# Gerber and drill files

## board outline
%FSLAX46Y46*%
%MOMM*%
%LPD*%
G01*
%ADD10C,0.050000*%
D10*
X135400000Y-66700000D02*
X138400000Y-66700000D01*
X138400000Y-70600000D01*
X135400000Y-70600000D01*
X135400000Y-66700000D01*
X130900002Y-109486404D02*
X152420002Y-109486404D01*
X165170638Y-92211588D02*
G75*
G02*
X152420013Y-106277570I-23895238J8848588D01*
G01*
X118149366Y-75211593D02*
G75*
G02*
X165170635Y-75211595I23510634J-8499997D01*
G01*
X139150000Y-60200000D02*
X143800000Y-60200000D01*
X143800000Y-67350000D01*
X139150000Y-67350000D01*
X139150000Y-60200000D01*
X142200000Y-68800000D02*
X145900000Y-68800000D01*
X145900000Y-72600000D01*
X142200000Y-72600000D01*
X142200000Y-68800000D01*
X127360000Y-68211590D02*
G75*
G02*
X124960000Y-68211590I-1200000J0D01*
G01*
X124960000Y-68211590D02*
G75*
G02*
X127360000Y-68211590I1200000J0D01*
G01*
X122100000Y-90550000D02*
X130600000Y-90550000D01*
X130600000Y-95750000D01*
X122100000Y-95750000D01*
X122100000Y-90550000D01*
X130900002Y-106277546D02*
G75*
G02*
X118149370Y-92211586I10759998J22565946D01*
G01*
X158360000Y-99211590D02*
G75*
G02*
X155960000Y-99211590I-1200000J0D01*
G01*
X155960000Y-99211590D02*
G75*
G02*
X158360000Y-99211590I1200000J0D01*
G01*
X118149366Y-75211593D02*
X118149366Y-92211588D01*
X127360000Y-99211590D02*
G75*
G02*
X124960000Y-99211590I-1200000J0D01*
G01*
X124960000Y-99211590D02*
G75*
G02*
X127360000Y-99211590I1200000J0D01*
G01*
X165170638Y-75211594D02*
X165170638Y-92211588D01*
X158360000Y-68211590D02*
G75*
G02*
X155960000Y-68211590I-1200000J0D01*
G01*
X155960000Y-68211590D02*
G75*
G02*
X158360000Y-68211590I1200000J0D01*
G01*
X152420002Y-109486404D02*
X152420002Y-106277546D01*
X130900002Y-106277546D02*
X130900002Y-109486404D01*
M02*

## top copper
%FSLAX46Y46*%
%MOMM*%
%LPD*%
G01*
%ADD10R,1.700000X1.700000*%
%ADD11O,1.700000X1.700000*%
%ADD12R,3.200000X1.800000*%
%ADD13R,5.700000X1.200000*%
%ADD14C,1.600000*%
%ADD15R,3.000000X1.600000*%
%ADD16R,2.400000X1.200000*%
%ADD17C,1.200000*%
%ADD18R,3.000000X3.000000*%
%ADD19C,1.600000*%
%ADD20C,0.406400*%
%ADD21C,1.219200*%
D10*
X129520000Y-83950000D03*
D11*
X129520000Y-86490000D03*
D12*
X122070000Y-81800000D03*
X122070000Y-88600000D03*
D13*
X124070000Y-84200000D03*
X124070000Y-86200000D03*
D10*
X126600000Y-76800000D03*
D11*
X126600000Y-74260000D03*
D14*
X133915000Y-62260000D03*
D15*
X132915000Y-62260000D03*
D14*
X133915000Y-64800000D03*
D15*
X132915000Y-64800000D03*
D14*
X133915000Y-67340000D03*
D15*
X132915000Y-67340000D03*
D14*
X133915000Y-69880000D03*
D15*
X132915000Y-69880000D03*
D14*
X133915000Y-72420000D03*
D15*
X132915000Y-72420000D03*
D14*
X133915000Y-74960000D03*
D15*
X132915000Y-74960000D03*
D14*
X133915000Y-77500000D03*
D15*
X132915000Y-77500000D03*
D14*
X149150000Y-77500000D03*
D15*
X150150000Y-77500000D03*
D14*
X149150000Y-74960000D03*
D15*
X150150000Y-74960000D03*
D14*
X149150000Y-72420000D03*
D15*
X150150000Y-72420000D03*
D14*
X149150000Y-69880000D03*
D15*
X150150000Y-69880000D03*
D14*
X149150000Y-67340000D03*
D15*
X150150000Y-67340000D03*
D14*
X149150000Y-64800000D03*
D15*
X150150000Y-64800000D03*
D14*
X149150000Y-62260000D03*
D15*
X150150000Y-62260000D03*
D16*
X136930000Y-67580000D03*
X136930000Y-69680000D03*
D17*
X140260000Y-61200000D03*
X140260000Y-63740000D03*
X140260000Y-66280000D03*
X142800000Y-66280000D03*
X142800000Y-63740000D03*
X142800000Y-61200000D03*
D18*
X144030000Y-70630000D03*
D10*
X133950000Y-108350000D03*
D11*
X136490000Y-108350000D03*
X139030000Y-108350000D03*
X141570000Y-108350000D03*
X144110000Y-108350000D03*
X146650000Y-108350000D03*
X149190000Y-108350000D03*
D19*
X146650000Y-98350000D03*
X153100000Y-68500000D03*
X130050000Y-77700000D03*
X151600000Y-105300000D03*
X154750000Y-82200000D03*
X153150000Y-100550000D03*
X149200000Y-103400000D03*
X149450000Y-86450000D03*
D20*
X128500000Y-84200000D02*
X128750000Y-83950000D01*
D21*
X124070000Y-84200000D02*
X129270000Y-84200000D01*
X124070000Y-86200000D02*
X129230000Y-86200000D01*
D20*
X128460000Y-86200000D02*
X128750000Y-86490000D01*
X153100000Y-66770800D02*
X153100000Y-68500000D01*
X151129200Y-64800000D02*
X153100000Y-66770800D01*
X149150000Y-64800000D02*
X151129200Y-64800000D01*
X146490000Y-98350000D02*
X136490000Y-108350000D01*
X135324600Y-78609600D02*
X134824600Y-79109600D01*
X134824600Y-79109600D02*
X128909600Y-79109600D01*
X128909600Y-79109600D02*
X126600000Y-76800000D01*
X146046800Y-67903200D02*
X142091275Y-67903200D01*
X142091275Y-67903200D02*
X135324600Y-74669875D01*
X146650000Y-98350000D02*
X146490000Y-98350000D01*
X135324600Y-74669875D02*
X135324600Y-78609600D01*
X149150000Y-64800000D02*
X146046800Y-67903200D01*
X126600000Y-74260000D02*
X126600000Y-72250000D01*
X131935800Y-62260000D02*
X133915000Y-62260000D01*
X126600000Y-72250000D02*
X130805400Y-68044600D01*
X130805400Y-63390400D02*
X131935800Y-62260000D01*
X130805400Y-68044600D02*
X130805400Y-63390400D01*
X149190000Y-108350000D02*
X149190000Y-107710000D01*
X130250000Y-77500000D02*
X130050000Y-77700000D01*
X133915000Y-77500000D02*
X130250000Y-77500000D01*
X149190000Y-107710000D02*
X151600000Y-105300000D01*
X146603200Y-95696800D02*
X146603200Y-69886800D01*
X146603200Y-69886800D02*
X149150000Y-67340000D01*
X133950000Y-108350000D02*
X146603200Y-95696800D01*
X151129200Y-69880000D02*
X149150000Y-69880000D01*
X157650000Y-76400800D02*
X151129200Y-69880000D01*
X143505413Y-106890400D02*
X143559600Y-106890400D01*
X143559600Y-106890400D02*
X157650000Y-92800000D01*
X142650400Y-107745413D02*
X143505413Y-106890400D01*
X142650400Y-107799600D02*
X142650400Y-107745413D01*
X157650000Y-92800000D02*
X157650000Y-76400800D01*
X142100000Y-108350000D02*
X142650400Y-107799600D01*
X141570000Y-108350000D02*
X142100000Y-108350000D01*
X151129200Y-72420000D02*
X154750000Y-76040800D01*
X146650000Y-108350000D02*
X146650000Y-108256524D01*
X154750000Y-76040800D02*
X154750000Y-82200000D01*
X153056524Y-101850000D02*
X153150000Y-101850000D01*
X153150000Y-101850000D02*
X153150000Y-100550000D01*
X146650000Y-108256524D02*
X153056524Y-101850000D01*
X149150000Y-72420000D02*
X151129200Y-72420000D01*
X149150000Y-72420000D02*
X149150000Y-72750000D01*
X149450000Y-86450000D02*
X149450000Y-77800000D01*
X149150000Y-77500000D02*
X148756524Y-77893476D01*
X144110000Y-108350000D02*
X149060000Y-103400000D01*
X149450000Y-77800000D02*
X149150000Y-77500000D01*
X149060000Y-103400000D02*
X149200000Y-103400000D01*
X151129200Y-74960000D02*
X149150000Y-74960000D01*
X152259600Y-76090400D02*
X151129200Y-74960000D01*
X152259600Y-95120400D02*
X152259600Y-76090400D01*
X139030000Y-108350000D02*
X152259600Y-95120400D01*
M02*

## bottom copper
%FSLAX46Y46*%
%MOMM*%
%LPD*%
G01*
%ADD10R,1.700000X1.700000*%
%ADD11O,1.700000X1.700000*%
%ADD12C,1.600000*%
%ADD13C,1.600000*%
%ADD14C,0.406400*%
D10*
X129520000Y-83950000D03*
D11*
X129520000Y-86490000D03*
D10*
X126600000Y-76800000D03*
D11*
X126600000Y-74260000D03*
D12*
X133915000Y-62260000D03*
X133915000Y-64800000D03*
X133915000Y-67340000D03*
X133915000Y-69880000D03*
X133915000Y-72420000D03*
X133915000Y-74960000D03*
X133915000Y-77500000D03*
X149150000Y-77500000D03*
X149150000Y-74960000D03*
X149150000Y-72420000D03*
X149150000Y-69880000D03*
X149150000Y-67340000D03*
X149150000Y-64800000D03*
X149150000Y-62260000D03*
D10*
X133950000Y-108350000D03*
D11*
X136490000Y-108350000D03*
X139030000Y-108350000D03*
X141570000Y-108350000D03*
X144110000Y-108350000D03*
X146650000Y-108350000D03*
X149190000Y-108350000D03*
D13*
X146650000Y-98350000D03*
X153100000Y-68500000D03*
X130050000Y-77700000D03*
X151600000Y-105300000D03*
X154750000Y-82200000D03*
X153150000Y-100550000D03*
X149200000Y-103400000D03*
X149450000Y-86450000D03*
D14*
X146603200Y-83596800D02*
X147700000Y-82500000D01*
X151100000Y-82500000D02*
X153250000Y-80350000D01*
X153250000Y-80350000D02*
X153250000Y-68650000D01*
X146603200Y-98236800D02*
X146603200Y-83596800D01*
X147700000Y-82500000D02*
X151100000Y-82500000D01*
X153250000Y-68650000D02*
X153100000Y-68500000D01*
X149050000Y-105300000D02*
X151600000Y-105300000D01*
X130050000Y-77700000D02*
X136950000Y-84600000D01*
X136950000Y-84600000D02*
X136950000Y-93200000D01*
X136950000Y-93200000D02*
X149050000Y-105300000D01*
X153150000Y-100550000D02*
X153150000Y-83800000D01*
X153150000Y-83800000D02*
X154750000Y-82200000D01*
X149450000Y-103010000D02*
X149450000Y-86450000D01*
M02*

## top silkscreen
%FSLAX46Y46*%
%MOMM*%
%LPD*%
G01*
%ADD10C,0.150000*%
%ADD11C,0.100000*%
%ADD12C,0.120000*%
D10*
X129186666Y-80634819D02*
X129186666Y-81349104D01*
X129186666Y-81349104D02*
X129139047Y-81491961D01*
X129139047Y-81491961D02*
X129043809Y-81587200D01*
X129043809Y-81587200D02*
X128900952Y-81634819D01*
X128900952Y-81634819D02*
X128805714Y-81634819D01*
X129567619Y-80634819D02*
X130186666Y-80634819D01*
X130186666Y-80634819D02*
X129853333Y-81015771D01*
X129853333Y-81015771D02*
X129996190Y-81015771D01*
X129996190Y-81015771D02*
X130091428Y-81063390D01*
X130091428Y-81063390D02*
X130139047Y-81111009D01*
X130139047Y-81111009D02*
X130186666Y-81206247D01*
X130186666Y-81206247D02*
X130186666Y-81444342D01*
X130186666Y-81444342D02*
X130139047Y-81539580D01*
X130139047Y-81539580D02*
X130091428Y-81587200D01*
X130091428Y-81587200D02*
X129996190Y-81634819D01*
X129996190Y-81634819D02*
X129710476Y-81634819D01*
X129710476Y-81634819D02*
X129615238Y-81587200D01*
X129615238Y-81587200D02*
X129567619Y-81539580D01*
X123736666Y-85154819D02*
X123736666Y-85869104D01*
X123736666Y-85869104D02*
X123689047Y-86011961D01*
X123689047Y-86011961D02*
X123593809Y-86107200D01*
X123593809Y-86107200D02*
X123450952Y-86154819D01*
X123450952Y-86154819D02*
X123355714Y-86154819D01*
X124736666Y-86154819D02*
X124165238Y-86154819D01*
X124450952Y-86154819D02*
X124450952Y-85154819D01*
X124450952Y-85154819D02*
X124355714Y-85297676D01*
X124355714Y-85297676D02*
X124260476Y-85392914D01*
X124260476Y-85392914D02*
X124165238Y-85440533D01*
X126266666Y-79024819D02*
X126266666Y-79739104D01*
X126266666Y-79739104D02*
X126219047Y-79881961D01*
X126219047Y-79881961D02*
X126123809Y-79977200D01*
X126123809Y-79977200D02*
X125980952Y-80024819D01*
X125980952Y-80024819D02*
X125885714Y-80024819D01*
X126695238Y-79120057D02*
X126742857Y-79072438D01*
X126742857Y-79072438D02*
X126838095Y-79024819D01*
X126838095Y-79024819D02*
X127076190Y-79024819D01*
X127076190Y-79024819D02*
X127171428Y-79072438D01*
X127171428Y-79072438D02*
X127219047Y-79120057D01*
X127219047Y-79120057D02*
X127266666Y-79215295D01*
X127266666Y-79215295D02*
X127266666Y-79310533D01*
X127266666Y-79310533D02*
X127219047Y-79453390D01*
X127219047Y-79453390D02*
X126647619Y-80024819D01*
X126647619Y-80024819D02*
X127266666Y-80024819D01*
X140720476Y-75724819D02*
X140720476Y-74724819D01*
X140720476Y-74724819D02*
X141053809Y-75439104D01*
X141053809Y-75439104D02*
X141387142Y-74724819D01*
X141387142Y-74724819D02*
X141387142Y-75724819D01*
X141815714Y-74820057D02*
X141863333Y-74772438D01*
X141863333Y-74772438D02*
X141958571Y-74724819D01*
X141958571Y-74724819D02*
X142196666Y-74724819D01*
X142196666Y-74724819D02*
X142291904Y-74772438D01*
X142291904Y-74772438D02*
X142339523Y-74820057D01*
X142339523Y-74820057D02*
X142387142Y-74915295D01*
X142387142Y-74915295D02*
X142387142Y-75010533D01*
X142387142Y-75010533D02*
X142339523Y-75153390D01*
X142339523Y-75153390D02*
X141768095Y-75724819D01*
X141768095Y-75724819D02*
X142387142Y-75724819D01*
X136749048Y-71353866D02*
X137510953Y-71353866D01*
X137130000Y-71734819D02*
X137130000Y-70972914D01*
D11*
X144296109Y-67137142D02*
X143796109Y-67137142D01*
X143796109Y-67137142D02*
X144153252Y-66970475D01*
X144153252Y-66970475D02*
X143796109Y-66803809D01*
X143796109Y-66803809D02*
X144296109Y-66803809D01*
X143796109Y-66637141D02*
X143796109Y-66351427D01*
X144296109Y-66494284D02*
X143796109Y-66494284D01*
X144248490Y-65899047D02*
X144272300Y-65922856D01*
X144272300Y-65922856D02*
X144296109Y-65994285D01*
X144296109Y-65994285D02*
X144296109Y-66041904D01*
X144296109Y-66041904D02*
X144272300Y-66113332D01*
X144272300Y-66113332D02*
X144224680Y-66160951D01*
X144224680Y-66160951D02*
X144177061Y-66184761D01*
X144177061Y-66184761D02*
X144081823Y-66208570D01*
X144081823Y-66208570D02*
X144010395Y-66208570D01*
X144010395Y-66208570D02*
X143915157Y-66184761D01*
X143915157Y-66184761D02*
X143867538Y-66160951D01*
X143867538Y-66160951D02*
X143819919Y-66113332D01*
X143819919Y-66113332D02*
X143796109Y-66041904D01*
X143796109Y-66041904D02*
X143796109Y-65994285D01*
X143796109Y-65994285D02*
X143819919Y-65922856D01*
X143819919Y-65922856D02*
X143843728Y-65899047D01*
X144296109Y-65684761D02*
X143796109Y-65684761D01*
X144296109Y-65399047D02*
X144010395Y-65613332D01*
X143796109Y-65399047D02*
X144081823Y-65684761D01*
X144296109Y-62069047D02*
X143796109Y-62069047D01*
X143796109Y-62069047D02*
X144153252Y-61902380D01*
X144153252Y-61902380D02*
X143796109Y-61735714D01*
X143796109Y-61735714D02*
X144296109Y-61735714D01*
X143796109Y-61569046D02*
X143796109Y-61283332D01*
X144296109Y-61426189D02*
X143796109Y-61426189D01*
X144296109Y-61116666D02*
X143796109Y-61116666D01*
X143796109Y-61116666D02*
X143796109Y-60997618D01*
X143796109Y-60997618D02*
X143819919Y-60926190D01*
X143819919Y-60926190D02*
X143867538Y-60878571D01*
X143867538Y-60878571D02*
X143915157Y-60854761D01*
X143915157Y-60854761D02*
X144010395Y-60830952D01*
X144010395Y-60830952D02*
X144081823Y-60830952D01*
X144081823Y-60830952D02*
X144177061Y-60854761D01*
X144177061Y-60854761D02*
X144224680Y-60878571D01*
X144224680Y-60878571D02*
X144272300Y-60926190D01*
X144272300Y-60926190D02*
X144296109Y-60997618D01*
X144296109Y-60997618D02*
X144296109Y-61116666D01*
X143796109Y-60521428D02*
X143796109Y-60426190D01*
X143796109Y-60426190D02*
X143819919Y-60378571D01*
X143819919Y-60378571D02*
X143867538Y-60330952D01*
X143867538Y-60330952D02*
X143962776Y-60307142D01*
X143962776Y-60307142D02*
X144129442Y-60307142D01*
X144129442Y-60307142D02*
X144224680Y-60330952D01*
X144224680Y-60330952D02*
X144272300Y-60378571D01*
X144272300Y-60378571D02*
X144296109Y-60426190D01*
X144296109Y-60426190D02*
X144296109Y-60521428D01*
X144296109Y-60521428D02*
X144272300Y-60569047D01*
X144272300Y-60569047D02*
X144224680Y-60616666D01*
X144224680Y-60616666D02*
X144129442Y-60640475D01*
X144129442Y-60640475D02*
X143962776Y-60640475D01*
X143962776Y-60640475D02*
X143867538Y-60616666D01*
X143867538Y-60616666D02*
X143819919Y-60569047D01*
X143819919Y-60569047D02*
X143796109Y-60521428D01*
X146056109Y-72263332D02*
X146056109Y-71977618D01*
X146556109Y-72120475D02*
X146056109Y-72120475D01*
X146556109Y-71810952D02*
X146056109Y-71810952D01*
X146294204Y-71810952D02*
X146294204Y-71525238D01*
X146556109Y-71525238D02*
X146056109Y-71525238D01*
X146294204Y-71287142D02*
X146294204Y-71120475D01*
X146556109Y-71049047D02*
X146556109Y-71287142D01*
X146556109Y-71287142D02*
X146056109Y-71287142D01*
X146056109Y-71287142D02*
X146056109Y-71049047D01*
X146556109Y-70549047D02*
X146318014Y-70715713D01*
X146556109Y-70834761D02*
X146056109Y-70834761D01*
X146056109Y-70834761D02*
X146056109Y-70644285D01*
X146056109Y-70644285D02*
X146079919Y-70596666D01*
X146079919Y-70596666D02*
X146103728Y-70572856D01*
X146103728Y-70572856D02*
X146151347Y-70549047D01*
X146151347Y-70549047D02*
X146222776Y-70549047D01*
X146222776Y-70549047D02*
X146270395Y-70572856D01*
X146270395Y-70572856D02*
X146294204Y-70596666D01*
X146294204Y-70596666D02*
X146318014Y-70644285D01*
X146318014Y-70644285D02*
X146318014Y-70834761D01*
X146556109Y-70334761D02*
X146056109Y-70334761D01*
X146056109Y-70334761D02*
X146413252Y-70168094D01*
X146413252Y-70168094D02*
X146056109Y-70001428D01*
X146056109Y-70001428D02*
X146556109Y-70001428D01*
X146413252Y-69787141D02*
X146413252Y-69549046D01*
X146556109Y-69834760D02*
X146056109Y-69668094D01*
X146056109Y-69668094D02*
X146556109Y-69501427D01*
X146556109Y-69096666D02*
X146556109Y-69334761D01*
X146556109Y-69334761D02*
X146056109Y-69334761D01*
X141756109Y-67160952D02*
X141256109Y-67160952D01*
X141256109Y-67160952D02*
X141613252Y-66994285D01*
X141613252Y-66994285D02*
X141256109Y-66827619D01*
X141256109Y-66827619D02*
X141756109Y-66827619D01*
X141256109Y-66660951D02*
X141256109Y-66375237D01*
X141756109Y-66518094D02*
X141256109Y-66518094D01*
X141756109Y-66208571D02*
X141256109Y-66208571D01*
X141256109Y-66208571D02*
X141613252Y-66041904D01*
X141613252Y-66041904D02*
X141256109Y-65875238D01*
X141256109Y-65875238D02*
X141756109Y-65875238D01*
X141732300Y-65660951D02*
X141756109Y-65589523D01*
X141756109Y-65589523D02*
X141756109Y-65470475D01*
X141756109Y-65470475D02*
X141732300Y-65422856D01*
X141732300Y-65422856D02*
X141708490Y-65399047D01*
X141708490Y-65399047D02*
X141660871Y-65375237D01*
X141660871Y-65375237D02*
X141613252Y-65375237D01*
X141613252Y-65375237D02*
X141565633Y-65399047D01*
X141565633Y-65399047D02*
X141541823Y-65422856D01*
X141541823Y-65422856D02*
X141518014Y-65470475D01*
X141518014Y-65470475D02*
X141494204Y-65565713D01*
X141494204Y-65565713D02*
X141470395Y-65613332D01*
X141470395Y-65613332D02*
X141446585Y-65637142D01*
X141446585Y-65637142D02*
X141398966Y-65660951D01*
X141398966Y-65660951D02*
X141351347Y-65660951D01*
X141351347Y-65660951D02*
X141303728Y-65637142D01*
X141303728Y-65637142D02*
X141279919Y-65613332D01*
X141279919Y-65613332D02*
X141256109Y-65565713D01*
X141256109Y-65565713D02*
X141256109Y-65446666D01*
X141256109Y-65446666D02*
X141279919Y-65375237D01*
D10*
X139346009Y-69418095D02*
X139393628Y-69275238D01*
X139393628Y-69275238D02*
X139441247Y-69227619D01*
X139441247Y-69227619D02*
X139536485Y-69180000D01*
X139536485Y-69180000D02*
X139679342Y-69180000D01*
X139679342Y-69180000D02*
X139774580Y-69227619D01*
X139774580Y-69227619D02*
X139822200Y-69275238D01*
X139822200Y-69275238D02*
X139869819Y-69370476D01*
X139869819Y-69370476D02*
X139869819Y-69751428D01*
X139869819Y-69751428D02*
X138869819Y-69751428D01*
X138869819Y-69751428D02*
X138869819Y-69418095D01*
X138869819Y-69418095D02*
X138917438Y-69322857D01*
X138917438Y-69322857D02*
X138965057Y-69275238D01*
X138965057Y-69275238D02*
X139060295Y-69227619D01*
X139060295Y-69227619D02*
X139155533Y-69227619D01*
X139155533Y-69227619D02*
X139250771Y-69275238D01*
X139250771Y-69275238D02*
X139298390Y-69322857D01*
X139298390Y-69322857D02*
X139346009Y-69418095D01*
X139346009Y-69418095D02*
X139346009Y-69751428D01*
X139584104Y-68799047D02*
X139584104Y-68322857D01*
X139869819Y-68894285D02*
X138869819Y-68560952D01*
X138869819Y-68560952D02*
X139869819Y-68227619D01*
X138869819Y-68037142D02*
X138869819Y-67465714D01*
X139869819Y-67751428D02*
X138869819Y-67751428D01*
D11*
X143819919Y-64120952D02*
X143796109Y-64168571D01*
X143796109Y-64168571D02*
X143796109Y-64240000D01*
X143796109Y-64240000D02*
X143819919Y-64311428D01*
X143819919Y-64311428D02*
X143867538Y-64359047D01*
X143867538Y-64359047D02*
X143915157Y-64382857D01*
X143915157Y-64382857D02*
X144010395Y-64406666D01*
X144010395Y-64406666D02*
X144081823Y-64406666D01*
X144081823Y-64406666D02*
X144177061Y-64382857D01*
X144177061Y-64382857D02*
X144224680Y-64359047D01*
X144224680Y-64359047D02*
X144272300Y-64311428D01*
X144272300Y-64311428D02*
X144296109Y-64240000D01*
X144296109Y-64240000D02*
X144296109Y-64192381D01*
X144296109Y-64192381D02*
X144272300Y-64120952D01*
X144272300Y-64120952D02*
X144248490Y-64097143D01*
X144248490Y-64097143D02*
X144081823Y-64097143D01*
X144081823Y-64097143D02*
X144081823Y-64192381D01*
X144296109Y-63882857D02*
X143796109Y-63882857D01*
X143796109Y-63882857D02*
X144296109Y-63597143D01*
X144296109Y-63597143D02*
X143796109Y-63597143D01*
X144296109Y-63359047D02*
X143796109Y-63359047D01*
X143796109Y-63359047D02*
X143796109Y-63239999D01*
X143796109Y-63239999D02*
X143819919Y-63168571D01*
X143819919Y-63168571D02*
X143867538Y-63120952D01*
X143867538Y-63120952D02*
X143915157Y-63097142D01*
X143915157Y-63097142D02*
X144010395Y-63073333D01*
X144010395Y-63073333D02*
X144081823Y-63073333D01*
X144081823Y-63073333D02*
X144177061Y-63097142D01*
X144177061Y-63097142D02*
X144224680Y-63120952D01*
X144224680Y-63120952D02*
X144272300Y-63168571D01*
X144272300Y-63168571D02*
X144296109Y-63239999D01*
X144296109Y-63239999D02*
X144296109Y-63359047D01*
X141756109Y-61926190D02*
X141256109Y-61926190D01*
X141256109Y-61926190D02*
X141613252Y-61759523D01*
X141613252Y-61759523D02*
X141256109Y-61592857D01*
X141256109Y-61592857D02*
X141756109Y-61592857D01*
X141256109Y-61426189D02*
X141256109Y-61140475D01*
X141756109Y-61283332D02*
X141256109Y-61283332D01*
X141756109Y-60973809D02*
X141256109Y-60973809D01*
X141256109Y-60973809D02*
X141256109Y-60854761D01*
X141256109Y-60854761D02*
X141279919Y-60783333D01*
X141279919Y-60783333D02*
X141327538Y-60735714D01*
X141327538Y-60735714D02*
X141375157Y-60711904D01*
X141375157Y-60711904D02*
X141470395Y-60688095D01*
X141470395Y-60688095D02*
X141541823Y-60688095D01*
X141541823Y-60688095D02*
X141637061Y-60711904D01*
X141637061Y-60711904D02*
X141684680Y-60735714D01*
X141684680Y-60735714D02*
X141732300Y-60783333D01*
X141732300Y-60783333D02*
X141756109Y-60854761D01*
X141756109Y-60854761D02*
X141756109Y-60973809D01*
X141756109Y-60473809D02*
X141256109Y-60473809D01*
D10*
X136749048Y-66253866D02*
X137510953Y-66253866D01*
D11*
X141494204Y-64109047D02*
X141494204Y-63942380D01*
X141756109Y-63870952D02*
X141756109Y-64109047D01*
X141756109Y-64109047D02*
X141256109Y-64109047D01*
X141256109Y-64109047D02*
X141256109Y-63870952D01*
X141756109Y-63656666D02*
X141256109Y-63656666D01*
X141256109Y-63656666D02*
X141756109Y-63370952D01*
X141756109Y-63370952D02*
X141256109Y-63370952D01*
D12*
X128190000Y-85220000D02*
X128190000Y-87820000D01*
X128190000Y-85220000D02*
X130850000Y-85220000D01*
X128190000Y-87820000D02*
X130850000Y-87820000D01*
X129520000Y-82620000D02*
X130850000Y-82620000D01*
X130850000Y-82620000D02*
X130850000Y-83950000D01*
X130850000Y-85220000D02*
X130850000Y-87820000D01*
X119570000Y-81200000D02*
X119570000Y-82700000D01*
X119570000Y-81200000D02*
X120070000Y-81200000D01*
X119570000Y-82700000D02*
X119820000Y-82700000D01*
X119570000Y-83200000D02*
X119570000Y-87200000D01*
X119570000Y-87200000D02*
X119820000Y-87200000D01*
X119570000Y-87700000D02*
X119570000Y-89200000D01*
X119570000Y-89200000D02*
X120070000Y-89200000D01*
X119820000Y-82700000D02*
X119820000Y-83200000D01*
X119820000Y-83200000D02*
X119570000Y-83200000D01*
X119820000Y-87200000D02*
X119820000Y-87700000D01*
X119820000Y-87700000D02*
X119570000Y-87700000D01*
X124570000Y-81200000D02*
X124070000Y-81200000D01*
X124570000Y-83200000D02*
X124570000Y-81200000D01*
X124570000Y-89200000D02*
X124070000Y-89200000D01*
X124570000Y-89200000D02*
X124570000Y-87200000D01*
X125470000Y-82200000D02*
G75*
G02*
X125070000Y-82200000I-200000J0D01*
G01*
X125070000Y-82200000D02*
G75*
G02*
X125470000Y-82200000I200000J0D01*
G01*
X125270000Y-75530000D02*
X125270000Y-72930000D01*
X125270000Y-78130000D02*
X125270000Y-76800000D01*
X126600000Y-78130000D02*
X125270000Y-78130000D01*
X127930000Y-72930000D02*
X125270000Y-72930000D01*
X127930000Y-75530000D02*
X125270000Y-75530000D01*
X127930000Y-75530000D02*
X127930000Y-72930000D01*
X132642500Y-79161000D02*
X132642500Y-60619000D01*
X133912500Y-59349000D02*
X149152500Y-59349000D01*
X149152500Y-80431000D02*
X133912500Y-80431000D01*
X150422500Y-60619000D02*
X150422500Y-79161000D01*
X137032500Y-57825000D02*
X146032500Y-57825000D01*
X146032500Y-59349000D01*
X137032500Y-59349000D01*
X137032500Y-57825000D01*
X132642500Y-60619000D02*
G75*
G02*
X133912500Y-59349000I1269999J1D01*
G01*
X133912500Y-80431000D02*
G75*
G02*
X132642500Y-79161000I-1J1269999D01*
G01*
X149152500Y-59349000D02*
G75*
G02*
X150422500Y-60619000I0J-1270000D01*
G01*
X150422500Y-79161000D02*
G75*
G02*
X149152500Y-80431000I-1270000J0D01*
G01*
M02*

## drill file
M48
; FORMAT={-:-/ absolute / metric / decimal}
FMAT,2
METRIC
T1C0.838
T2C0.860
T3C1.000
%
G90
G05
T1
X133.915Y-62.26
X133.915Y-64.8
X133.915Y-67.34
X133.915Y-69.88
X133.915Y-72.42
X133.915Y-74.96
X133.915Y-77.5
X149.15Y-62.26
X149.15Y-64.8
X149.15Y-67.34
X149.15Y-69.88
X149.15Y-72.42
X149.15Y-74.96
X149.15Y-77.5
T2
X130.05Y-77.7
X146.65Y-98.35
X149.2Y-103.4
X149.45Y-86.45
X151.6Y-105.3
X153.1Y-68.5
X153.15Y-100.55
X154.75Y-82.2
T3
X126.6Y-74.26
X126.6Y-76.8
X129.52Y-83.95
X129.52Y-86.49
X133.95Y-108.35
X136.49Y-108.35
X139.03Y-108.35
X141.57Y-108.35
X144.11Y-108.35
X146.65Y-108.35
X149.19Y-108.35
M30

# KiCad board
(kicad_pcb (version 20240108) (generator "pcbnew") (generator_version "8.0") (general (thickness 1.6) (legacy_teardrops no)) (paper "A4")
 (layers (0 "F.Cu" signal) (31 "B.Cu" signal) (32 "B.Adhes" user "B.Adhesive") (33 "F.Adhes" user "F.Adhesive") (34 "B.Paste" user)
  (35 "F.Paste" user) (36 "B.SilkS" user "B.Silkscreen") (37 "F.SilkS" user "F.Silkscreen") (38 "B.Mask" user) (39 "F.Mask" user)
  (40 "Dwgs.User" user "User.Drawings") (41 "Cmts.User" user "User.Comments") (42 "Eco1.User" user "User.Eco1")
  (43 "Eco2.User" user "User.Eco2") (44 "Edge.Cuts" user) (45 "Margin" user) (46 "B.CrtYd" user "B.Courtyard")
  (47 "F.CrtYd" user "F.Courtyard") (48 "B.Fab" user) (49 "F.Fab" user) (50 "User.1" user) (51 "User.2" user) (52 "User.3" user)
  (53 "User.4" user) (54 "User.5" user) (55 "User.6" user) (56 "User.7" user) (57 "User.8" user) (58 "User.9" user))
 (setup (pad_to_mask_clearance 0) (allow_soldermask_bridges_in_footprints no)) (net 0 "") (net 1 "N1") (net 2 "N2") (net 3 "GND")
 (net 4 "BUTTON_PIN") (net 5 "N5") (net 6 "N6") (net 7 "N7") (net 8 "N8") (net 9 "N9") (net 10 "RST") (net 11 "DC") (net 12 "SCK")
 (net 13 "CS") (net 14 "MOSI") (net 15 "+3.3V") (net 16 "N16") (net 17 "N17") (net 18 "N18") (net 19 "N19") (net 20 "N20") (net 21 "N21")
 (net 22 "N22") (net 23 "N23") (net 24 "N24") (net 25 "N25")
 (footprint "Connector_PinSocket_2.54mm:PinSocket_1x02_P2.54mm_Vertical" (layer "F.Cu") (at 129.52 83.95)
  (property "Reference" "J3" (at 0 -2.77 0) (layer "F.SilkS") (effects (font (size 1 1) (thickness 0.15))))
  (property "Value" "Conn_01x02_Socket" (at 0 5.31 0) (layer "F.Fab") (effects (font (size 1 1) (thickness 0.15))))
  (fp_line (start -1.33 1.27) (end -1.33 3.87) (stroke (width 0.12) (type solid)) (layer "F.SilkS"))
  (fp_line (start -1.33 1.27) (end 1.33 1.27) (stroke (width 0.12) (type solid)) (layer "F.SilkS"))
  (fp_line (start -1.33 3.87) (end 1.33 3.87) (stroke (width 0.12) (type solid)) (layer "F.SilkS"))
  (fp_line (start 0 -1.33) (end 1.33 -1.33) (stroke (width 0.12) (type solid)) (layer "F.SilkS"))
  (fp_line (start 1.33 -1.33) (end 1.33 0) (stroke (width 0.12) (type solid)) (layer "F.SilkS"))
  (fp_line (start 1.33 1.27) (end 1.33 3.87) (stroke (width 0.12) (type solid)) (layer "F.SilkS"))
  (pad "1" thru_hole rect (at 0 0) (size 1.7 1.7) (drill 1) (layers "*.Cu" "*.Mask") (remove_unused_layers no) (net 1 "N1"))
  (pad "2" thru_hole oval (at 0 2.54) (size 1.7 1.7) (drill 1) (layers "*.Cu" "*.Mask") (remove_unused_layers no) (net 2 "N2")))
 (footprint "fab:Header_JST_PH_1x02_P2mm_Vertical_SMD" (layer "F.Cu") (at 124.07 85.2)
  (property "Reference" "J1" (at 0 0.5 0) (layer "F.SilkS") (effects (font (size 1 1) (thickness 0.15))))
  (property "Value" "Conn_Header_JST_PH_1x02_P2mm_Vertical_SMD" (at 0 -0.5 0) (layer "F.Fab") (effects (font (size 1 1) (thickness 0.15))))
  (fp_line (start -4.5 -4) (end -4.5 -2.5) (stroke (width 0.12) (type solid)) (layer "F.SilkS"))
  (fp_line (start -4.5 -4) (end -4 -4) (stroke (width 0.12) (type solid)) (layer "F.SilkS"))
  (fp_line (start -4.5 -2.5) (end -4.25 -2.5) (stroke (width 0.12) (type solid)) (layer "F.SilkS"))
  (fp_line (start -4.5 -2) (end -4.5 2) (stroke (width 0.12) (type solid)) (layer "F.SilkS"))
  (fp_line (start -4.5 2) (end -4.25 2) (stroke (width 0.12) (type solid)) (layer "F.SilkS"))
  (fp_line (start -4.5 2.5) (end -4.5 4) (stroke (width 0.12) (type solid)) (layer "F.SilkS"))
  (fp_line (start -4.5 4) (end -4 4) (stroke (width 0.12) (type solid)) (layer "F.SilkS"))
  (fp_line (start -4.25 -2.5) (end -4.25 -2) (stroke (width 0.12) (type solid)) (layer "F.SilkS"))
  (fp_line (start -4.25 -2) (end -4.5 -2) (stroke (width 0.12) (type solid)) (layer "F.SilkS"))
  (fp_line (start -4.25 2) (end -4.25 2.5) (stroke (width 0.12) (type solid)) (layer "F.SilkS"))
  (fp_line (start -4.25 2.5) (end -4.5 2.5) (stroke (width 0.12) (type solid)) (layer "F.SilkS"))
  (fp_line (start 0.5 -4) (end 0 -4) (stroke (width 0.12) (type solid)) (layer "F.SilkS"))
  (fp_line (start 0.5 -2) (end 0.5 -4) (stroke (width 0.12) (type solid)) (layer "F.SilkS"))
  (fp_line (start 0.5 4) (end 0 4) (stroke (width 0.12) (type solid)) (layer "F.SilkS"))
  (fp_line (start 0.5 4) (end 0.5 2) (stroke (width 0.12) (type solid)) (layer "F.SilkS"))
  (fp_circle (center 1.2 -3) (end 1.4 -3) (stroke (width 0.12) (type solid)) (fill none) (layer "F.SilkS"))
  (pad "" smd rect (at -2 -3.4) (size 3.2 1.8) (layers "F.Cu" "F.Paste" "F.Mask"))
  (pad "" smd rect (at -2 3.4) (size 3.2 1.8) (layers "F.Cu" "F.Paste" "F.Mask"))
  (pad "1" smd rect (at 0 -1) (size 5.7 1.2) (layers "F.Cu" "F.Paste" "F.Mask") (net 1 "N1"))
  (pad "2" smd rect (at 0 1) (size 5.7 1.2) (layers "F.Cu" "F.Paste" "F.Mask") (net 2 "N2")))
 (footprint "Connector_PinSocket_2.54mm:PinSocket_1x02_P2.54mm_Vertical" (layer "F.Cu") (at 126.6 76.8 180)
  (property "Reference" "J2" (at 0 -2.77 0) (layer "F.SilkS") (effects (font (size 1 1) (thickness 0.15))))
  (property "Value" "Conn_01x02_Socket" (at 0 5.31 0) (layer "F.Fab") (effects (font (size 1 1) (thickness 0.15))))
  (fp_line (start 1.33 1.27) (end 1.33 3.87) (stroke (width 0.12) (type solid)) (layer "F.SilkS"))
  (fp_line (start 1.33 -1.33) (end 1.33 0) (stroke (width 0.12) (type solid)) (layer "F.SilkS"))
  (fp_line (start 0 -1.33) (end 1.33 -1.33) (stroke (width 0.12) (type solid)) (layer "F.SilkS"))
  (fp_line (start -1.33 3.87) (end 1.33 3.87) (stroke (width 0.12) (type solid)) (layer "F.SilkS"))
  (fp_line (start -1.33 1.27) (end 1.33 1.27) (stroke (width 0.12) (type solid)) (layer "F.SilkS"))
  (fp_line (start -1.33 1.27) (end -1.33 3.87) (stroke (width 0.12) (type solid)) (layer "F.SilkS"))
  (pad "1" thru_hole rect (at 0 0 180) (size 1.7 1.7) (drill 1) (layers "*.Cu" "*.Mask") (remove_unused_layers no) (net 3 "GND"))
  (pad "2" thru_hole oval (at 0 2.54 180) (size 1.7 1.7) (drill 1) (layers "*.Cu" "*.Mask") (remove_unused_layers no) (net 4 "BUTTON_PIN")))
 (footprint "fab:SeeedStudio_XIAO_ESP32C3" (layer "F.Cu") (at 141.53 69.88)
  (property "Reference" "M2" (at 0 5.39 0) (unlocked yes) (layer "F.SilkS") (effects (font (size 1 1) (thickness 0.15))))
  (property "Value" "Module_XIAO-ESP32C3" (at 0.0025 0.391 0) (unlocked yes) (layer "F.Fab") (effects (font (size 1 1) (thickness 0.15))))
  (fp_line (start -8.8875 9.281) (end -8.8875 -9.261) (stroke (width 0.12) (type solid)) (layer "F.SilkS"))
  (fp_line (start -7.6175 -10.531) (end 7.6225 -10.531) (stroke (width 0.12) (type solid)) (layer "F.SilkS"))
  (fp_line (start 7.6225 10.551) (end -7.6175 10.551) (stroke (width 0.12) (type solid)) (layer "F.SilkS"))
  (fp_line (start 8.8925 -9.261) (end 8.8925 9.281) (stroke (width 0.12) (type solid)) (layer "F.SilkS"))
  (fp_rect (start -4.4975 -10.531) (end 4.5025 -12.055) (stroke (width 0.12) (type solid)) (fill none) (layer "F.SilkS"))
  (fp_arc (start -8.8875 -9.261) (mid -8.515526 -10.159026) (end -7.6175 -10.531) (stroke (width 0.12) (type solid)) (layer "F.SilkS"))
  (fp_arc (start -7.6175 10.551) (mid -8.515526 10.179026) (end -8.8875 9.281) (stroke (width 0.12) (type solid)) (layer "F.SilkS"))
  (fp_arc (start 7.6225 -10.531) (mid 8.520526 -10.159026) (end 8.8925 -9.261) (stroke (width 0.12) (type solid)) (layer "F.SilkS"))
  (fp_arc (start 8.8925 9.281) (mid 8.520526 10.179026) (end 7.6225 10.551) (stroke (width 0.12) (type solid)) (layer "F.SilkS"))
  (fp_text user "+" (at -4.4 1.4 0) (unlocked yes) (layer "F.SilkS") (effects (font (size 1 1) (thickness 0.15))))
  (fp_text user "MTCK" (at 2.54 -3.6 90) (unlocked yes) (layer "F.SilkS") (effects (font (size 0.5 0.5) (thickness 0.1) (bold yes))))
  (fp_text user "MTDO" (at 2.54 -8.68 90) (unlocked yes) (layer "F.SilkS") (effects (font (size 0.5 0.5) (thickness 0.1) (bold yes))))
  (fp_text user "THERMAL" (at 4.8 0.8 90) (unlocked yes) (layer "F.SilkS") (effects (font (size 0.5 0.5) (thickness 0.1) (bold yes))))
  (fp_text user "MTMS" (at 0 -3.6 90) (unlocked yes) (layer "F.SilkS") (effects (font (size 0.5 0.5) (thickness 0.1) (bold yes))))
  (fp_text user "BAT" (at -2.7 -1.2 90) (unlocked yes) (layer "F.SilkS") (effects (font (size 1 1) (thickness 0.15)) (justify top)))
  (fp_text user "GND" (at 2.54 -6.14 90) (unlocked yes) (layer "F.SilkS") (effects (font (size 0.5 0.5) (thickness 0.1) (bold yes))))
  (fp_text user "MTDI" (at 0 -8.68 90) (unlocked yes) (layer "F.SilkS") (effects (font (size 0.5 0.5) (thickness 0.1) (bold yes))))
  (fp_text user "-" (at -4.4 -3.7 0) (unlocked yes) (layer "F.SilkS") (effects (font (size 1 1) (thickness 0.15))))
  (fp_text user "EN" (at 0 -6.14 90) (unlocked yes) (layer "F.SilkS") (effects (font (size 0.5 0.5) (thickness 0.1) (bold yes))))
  (pad "1" thru_hole circle (at -7.615 -7.62) (size 1.6 1.6) (drill 0.8382) (layers "*.Cu" "*.Mask") (remove_unused_layers no)
   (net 4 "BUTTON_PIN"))
  (pad "1" smd rect (at -7.615 -7.62) (size 3 1.6) (drill (offset -1 0)) (layers "F.Cu" "F.Paste" "F.Mask") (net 4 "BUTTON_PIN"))
  (pad "2" thru_hole circle (at -7.615 -5.08) (size 1.6 1.6) (drill 0.8382) (layers "*.Cu" "*.Mask") (remove_unused_layers no) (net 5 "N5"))
  (pad "2" smd rect (at -7.615 -5.08) (size 3 1.6) (drill (offset -1 0)) (layers "F.Cu" "F.Paste" "F.Mask") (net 5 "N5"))
  (pad "3" thru_hole circle (at -7.615 -2.54) (size 1.6 1.6) (drill 0.8382) (layers "*.Cu" "*.Mask") (remove_unused_layers no) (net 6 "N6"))
  (pad "3" smd rect (at -7.615 -2.54) (size 3 1.6) (drill (offset -1 0)) (layers "F.Cu" "F.Paste" "F.Mask") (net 6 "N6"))
  (pad "4" thru_hole circle (at -7.615 0) (size 1.6 1.6) (drill 0.8382) (layers "*.Cu" "*.Mask") (remove_unused_layers no) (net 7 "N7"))
  (pad "4" smd rect (at -7.615 0) (size 3 1.6) (drill (offset -1 0)) (layers "F.Cu" "F.Paste" "F.Mask") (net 7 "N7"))
  (pad "5" thru_hole circle (at -7.615 2.54) (size 1.6 1.6) (drill 0.8382) (layers "*.Cu" "*.Mask") (remove_unused_layers no) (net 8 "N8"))
  (pad "5" smd rect (at -7.615 2.54) (size 3 1.6) (drill (offset -1 0)) (layers "F.Cu" "F.Paste" "F.Mask") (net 8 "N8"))
  (pad "6" thru_hole circle (at -7.615 5.08) (size 1.6 1.6) (drill 0.8382) (layers "*.Cu" "*.Mask") (remove_unused_layers no) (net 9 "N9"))
  (pad "6" smd rect (at -7.615 5.08) (size 3 1.6) (drill (offset -1 0)) (layers "F.Cu" "F.Paste" "F.Mask") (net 9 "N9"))
  (pad "7" thru_hole circle (at -7.615 7.62) (size 1.6 1.6) (drill 0.8382) (layers "*.Cu" "*.Mask") (remove_unused_layers no) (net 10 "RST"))
  (pad "7" smd rect (at -7.615 7.62) (size 3 1.6) (drill (offset -1 0)) (layers "F.Cu" "F.Paste" "F.Mask") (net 10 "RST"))
  (pad "8" thru_hole circle (at 7.62 7.62) (size 1.6 1.6) (drill 0.8382) (layers "*.Cu" "*.Mask") (remove_unused_layers no) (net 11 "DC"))
  (pad "8" smd rect (at 7.62 7.62) (size 3 1.6) (drill (offset 1 0)) (layers "F.Cu" "F.Paste" "F.Mask") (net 11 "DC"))
  (pad "9" thru_hole circle (at 7.62 5.08) (size 1.6 1.6) (drill 0.8382) (layers "*.Cu" "*.Mask") (remove_unused_layers no) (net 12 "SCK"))
  (pad "9" smd rect (at 7.62 5.08) (size 3 1.6) (drill (offset 1 0)) (layers "F.Cu" "F.Paste" "F.Mask") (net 12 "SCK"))
  (pad "10" thru_hole circle (at 7.62 2.54) (size 1.6 1.6) (drill 0.8382) (layers "*.Cu" "*.Mask") (remove_unused_layers no) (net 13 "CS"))
  (pad "10" smd rect (at 7.62 2.54) (size 3 1.6) (drill (offset 1 0)) (layers "F.Cu" "F.Paste" "F.Mask") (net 13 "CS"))
  (pad "11" thru_hole circle (at 7.62 0) (size 1.6 1.6) (drill 0.8382) (layers "*.Cu" "*.Mask") (remove_unused_layers no) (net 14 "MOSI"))
  (pad "11" smd rect (at 7.62 0) (size 3 1.6) (drill (offset 1 0)) (layers "F.Cu" "F.Paste" "F.Mask") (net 14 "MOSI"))
  (pad "12" thru_hole circle (at 7.62 -2.54) (size 1.6 1.6) (drill 0.8382) (layers "*.Cu" "*.Mask") (remove_unused_layers no)
   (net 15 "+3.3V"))
  (pad "12" smd rect (at 7.62 -2.54) (size 3 1.6) (drill (offset 1 0)) (layers "F.Cu" "F.Paste" "F.Mask") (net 15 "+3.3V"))
  (pad "13" thru_hole circle (at 7.62 -5.08) (size 1.6 1.6) (drill 0.8382) (layers "*.Cu" "*.Mask") (remove_unused_layers no) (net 3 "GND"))
  (pad "13" smd rect (at 7.62 -5.08) (size 3 1.6) (drill (offset 1 0)) (layers "F.Cu" "F.Paste" "F.Mask") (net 3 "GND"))
  (pad "14" thru_hole circle (at 7.62 -7.62) (size 1.6 1.6) (drill 0.8382) (layers "*.Cu" "*.Mask") (remove_unused_layers no) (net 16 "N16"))
  (pad "14" smd rect (at 7.62 -7.62) (size 3 1.6) (drill (offset 1 0)) (layers "F.Cu" "F.Paste" "F.Mask") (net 16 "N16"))
  (pad "15" smd rect (at -4.6 -2.3) (size 2.4 1.2) (layers "F.Cu" "F.Paste" "F.Mask") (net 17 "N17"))
  (pad "16" smd rect (at -4.6 -0.2) (size 2.4 1.2) (layers "F.Cu" "F.Paste" "F.Mask") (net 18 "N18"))
  (pad "17" smd circle (at -1.27 -8.68) (size 1.2 1.2) (layers "F.Cu" "F.Paste" "F.Mask") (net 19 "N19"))
  (pad "18" smd circle (at -1.27 -6.14) (size 1.2 1.2) (layers "F.Cu" "F.Paste" "F.Mask") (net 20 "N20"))
  (pad "19" smd circle (at -1.27 -3.6) (size 1.2 1.2) (layers "F.Cu" "F.Paste" "F.Mask") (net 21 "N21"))
  (pad "20" smd circle (at 1.27 -3.6) (size 1.2 1.2) (layers "F.Cu" "F.Paste" "F.Mask") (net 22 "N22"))
  (pad "21" smd circle (at 1.27 -6.14) (size 1.2 1.2) (layers "F.Cu" "F.Paste" "F.Mask") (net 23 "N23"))
  (pad "22" smd circle (at 1.27 -8.68) (size 1.2 1.2) (layers "F.Cu" "F.Paste" "F.Mask") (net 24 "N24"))
  (pad "23" smd rect (at 2.5 0.75) (size 3 3) (layers "F.Cu" "F.Paste" "F.Mask") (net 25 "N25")))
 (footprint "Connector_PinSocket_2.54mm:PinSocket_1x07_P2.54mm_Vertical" (layer "B.Cu") (at 133.95 108.35 -90)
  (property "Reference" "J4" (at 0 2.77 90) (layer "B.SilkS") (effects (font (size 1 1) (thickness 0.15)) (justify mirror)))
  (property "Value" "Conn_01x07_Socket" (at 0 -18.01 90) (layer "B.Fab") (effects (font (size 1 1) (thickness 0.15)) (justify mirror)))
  (pad "1" thru_hole rect (at 0 0 270) (size 1.7 1.7) (drill 1) (layers "*.Cu" "*.Mask") (remove_unused_layers no) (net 15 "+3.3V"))
  (pad "2" thru_hole oval (at 0 -2.54 270) (size 1.7 1.7) (drill 1) (layers "*.Cu" "*.Mask") (remove_unused_layers no) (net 3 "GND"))
  (pad "3" thru_hole oval (at 0 -5.08 270) (size 1.7 1.7) (drill 1) (layers "*.Cu" "*.Mask") (remove_unused_layers no) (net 12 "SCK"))
  (pad "4" thru_hole oval (at 0 -7.62 270) (size 1.7 1.7) (drill 1) (layers "*.Cu" "*.Mask") (remove_unused_layers no) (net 14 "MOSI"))
  (pad "5" thru_hole oval (at 0 -10.16 270) (size 1.7 1.7) (drill 1) (layers "*.Cu" "*.Mask") (remove_unused_layers no) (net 11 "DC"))
  (pad "6" thru_hole oval (at 0 -12.7 270) (size 1.7 1.7) (drill 1) (layers "*.Cu" "*.Mask") (remove_unused_layers no) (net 13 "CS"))
  (pad "7" thru_hole oval (at 0 -15.24 270) (size 1.7 1.7) (drill 1) (layers "*.Cu" "*.Mask") (remove_unused_layers no) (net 10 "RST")))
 (gr_rect (start 135.4 66.7) (end 138.4 70.6) (stroke (width 0.05) (type default)) (fill none) (layer "Edge.Cuts"))
 (gr_line (start 130.900002 109.486404) (end 152.420002 109.486404) (stroke (width 0.05) (type default)) (layer "Edge.Cuts"))
 (gr_arc (start 165.170638 92.211588) (mid 160.154238 100.476411) (end 152.420002 106.277546) (stroke (width 0.05) (type default))
  (layer "Edge.Cuts"))
 (gr_arc (start 118.149366 75.211593) (mid 141.660002 58.71159) (end 165.170638 75.211594) (stroke (width 0.05) (type default))
  (layer "Edge.Cuts"))
 (gr_rect (start 139.15 60.2) (end 143.8 67.35) (stroke (width 0.05) (type default)) (fill none) (layer "Edge.Cuts"))
 (gr_rect (start 142.2 68.8) (end 145.9 72.6) (stroke (width 0.05) (type default)) (fill none) (layer "Edge.Cuts"))
 (gr_circle (center 126.16 68.21159) (end 127.36 68.21159) (stroke (width 0.05) (type default)) (fill none) (layer "Edge.Cuts"))
 (gr_rect (start 122.1 90.55) (end 130.6 95.75) (stroke (width 0.05) (type default)) (fill none) (layer "Edge.Cuts"))
 (gr_arc (start 130.900002 106.277546) (mid 123.137531 100.502006) (end 118.149366 92.211588) (stroke (width 0.05) (type default))
  (layer "Edge.Cuts"))
 (gr_circle (center 157.16 99.21159) (end 158.36 99.21159) (stroke (width 0.05) (type default)) (fill none) (layer "Edge.Cuts"))
 (gr_line (start 118.149366 75.211593) (end 118.149366 92.211588) (stroke (width 0.05) (type default)) (layer "Edge.Cuts"))
 (gr_circle (center 126.16 99.21159) (end 127.36 99.21159) (stroke (width 0.05) (type default)) (fill none) (layer "Edge.Cuts"))
 (gr_line (start 165.170638 75.211594) (end 165.170638 92.211588) (stroke (width 0.05) (type default)) (layer "Edge.Cuts"))
 (gr_circle (center 157.16 68.21159) (end 158.36 68.21159) (stroke (width 0.05) (type default)) (fill none) (layer "Edge.Cuts"))
 (gr_line (start 152.420002 109.486404) (end 152.420002 106.277546) (stroke (width 0.05) (type default)) (layer "Edge.Cuts"))
 (gr_line (start 130.900002 106.277546) (end 130.900002 109.486404) (stroke (width 0.05) (type default)) (layer "Edge.Cuts"))
 (segment (start 128.5 84.2) (end 128.75 83.95) (width 0.4064) (layer "F.Cu") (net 1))
 (segment (start 124.07 84.2) (end 129.27 84.2) (width 1.2192) (layer "F.Cu") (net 1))
 (segment (start 124.07 86.2) (end 129.23 86.2) (width 1.2192) (layer "F.Cu") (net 2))
 (segment (start 128.46 86.2) (end 128.75 86.49) (width 0.4064) (layer "F.Cu") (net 2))
 (segment (start 153.1 66.7708) (end 153.1 68.5) (width 0.4064) (layer "F.Cu") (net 3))
 (segment (start 151.1292 64.8) (end 153.1 66.7708) (width 0.4064) (layer "F.Cu") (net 3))
 (segment (start 149.15 64.8) (end 151.1292 64.8) (width 0.4064) (layer "F.Cu") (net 3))
 (segment (start 146.49 98.35) (end 136.49 108.35) (width 0.4064) (layer "F.Cu") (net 3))
 (segment (start 135.3246 78.6096) (end 134.8246 79.1096) (width 0.4064) (layer "F.Cu") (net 3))
 (segment (start 134.8246 79.1096) (end 128.9096 79.1096) (width 0.4064) (layer "F.Cu") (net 3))
 (segment (start 128.9096 79.1096) (end 126.6 76.8) (width 0.4064) (layer "F.Cu") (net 3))
 (segment (start 146.0468 67.9032) (end 142.091275 67.9032) (width 0.4064) (layer "F.Cu") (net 3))
 (segment (start 142.091275 67.9032) (end 135.3246 74.669875) (width 0.4064) (layer "F.Cu") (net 3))
 (segment (start 146.65 98.35) (end 146.49 98.35) (width 0.4064) (layer "F.Cu") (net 3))
 (segment (start 135.3246 74.669875) (end 135.3246 78.6096) (width 0.4064) (layer "F.Cu") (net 3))
 (segment (start 149.15 64.8) (end 146.0468 67.9032) (width 0.4064) (layer "F.Cu") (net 3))
 (via (at 146.65 98.35) (size 1.6) (drill 0.86) (layers "F.Cu" "B.Cu") (free yes) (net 3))
 (via (at 153.1 68.5) (size 1.6) (drill 0.86) (layers "F.Cu" "B.Cu") (free yes) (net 3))
 (segment (start 146.6032 83.5968) (end 147.7 82.5) (width 0.4064) (layer "B.Cu") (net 3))
 (segment (start 151.1 82.5) (end 153.25 80.35) (width 0.4064) (layer "B.Cu") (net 3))
 (segment (start 153.25 80.35) (end 153.25 68.65) (width 0.4064) (layer "B.Cu") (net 3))
 (segment (start 146.6032 98.2368) (end 146.6032 83.5968) (width 0.4064) (layer "B.Cu") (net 3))
 (segment (start 147.7 82.5) (end 151.1 82.5) (width 0.4064) (layer "B.Cu") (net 3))
 (segment (start 153.25 68.65) (end 153.1 68.5) (width 0.4064) (layer "B.Cu") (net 3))
 (segment (start 126.6 74.26) (end 126.6 72.25) (width 0.4064) (layer "F.Cu") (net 4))
 (segment (start 131.9358 62.26) (end 133.915 62.26) (width 0.4064) (layer "F.Cu") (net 4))
 (segment (start 126.6 72.25) (end 130.8054 68.0446) (width 0.4064) (layer "F.Cu") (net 4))
 (segment (start 130.8054 63.3904) (end 131.9358 62.26) (width 0.4064) (layer "F.Cu") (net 4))
 (segment (start 130.8054 68.0446) (end 130.8054 63.3904) (width 0.4064) (layer "F.Cu") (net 4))
 (segment (start 149.19 108.35) (end 149.19 107.71) (width 0.4064) (layer "F.Cu") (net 10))
 (segment (start 130.25 77.5) (end 130.05 77.7) (width 0.4064) (layer "F.Cu") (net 10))
 (segment (start 133.915 77.5) (end 130.25 77.5) (width 0.4064) (layer "F.Cu") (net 10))
 (segment (start 149.19 107.71) (end 151.6 105.3) (width 0.4064) (layer "F.Cu") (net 10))
 (via (at 130.05 77.7) (size 1.6) (drill 0.86) (layers "F.Cu" "B.Cu") (free yes) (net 10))
 (via (at 151.6 105.3) (size 1.6) (drill 0.86) (layers "F.Cu" "B.Cu") (free yes) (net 10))
 (segment (start 149.05 105.3) (end 151.6 105.3) (width 0.4064) (layer "B.Cu") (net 10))
 (segment (start 130.05 77.7) (end 136.95 84.6) (width 0.4064) (layer "B.Cu") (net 10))
 (segment (start 136.95 84.6) (end 136.95 93.2) (width 0.4064) (layer "B.Cu") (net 10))
 (segment (start 136.95 93.2) (end 149.05 105.3) (width 0.4064) (layer "B.Cu") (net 10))
 (segment (start 146.6032 95.6968) (end 146.6032 69.8868) (width 0.4064) (layer "F.Cu") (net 15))
 (segment (start 146.6032 69.8868) (end 149.15 67.34) (width 0.4064) (layer "F.Cu") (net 15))
 (segment (start 133.95 108.35) (end 146.6032 95.6968) (width 0.4064) (layer "F.Cu") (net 15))
 (segment (start 151.1292 69.88) (end 149.15 69.88) (width 0.4064) (layer "F.Cu") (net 14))
 (segment (start 157.65 76.4008) (end 151.1292 69.88) (width 0.4064) (layer "F.Cu") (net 14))
 (segment (start 143.505413 106.8904) (end 143.5596 106.8904) (width 0.4064) (layer "F.Cu") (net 14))
 (segment (start 143.5596 106.8904) (end 157.65 92.8) (width 0.4064) (layer "F.Cu") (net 14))
 (segment (start 142.6504 107.745413) (end 143.505413 106.8904) (width 0.4064) (layer "F.Cu") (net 14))
 (segment (start 142.6504 107.7996) (end 142.6504 107.745413) (width 0.4064) (layer "F.Cu") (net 14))
 (segment (start 157.65 92.8) (end 157.65 76.4008) (width 0.4064) (layer "F.Cu") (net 14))
 (segment (start 142.1 108.35) (end 142.6504 107.7996) (width 0.4064) (layer "F.Cu") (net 14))
 (segment (start 141.57 108.35) (end 142.1 108.35) (width 0.4064) (layer "F.Cu") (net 14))
 (segment (start 151.1292 72.42) (end 154.75 76.0408) (width 0.4064) (layer "F.Cu") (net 13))
 (segment (start 146.65 108.35) (end 146.65 108.256524) (width 0.4064) (layer "F.Cu") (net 13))
 (segment (start 154.75 76.0408) (end 154.75 82.2) (width 0.4064) (layer "F.Cu") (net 13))
 (segment (start 153.056524 101.85) (end 153.15 101.85) (width 0.4064) (layer "F.Cu") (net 13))
 (segment (start 153.15 101.85) (end 153.15 100.55) (width 0.4064) (layer "F.Cu") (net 13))
 (segment (start 146.65 108.256524) (end 153.056524 101.85) (width 0.4064) (layer "F.Cu") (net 13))
 (segment (start 149.15 72.42) (end 151.1292 72.42) (width 0.4064) (layer "F.Cu") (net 13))
 (segment (start 149.15 72.42) (end 149.15 72.75) (width 0.4064) (layer "F.Cu") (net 13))
 (via (at 154.75 82.2) (size 1.6) (drill 0.86) (layers "F.Cu" "B.Cu") (free yes) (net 13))
 (via (at 153.15 100.55) (size 1.6) (drill 0.86) (layers "F.Cu" "B.Cu") (free yes) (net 13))
 (segment (start 153.15 100.55) (end 153.15 83.8) (width 0.4064) (layer "B.Cu") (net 13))
 (segment (start 153.15 83.8) (end 154.75 82.2) (width 0.4064) (layer "B.Cu") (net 13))
 (segment (start 149.45 86.45) (end 149.45 77.8) (width 0.4064) (layer "F.Cu") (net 11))
 (segment (start 149.15 77.5) (end 148.756524 77.893476) (width 0.4064) (layer "F.Cu") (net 11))
 (segment (start 144.11 108.35) (end 149.06 103.4) (width 0.4064) (layer "F.Cu") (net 11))
 (segment (start 149.45 77.8) (end 149.15 77.5) (width 0.4064) (layer "F.Cu") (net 11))
 (segment (start 149.06 103.4) (end 149.2 103.4) (width 0.4064) (layer "F.Cu") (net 11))
 (via (at 149.2 103.4) (size 1.6) (drill 0.86) (layers "F.Cu" "B.Cu") (free yes) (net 11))
 (via (at 149.45 86.45) (size 1.6) (drill 0.86) (layers "F.Cu" "B.Cu") (free yes) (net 11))
 (segment (start 149.45 103.01) (end 149.45 86.45) (width 0.4064) (layer "B.Cu") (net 11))
 (segment (start 151.1292 74.96) (end 149.15 74.96) (width 0.4064) (layer "F.Cu") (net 12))
 (segment (start 152.2596 76.0904) (end 151.1292 74.96) (width 0.4064) (layer "F.Cu") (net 12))
 (segment (start 152.2596 95.1204) (end 152.2596 76.0904) (width 0.4064) (layer "F.Cu") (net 12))
 (segment (start 139.03 108.35) (end 152.2596 95.1204) (width 0.4064) (layer "F.Cu") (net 12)))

